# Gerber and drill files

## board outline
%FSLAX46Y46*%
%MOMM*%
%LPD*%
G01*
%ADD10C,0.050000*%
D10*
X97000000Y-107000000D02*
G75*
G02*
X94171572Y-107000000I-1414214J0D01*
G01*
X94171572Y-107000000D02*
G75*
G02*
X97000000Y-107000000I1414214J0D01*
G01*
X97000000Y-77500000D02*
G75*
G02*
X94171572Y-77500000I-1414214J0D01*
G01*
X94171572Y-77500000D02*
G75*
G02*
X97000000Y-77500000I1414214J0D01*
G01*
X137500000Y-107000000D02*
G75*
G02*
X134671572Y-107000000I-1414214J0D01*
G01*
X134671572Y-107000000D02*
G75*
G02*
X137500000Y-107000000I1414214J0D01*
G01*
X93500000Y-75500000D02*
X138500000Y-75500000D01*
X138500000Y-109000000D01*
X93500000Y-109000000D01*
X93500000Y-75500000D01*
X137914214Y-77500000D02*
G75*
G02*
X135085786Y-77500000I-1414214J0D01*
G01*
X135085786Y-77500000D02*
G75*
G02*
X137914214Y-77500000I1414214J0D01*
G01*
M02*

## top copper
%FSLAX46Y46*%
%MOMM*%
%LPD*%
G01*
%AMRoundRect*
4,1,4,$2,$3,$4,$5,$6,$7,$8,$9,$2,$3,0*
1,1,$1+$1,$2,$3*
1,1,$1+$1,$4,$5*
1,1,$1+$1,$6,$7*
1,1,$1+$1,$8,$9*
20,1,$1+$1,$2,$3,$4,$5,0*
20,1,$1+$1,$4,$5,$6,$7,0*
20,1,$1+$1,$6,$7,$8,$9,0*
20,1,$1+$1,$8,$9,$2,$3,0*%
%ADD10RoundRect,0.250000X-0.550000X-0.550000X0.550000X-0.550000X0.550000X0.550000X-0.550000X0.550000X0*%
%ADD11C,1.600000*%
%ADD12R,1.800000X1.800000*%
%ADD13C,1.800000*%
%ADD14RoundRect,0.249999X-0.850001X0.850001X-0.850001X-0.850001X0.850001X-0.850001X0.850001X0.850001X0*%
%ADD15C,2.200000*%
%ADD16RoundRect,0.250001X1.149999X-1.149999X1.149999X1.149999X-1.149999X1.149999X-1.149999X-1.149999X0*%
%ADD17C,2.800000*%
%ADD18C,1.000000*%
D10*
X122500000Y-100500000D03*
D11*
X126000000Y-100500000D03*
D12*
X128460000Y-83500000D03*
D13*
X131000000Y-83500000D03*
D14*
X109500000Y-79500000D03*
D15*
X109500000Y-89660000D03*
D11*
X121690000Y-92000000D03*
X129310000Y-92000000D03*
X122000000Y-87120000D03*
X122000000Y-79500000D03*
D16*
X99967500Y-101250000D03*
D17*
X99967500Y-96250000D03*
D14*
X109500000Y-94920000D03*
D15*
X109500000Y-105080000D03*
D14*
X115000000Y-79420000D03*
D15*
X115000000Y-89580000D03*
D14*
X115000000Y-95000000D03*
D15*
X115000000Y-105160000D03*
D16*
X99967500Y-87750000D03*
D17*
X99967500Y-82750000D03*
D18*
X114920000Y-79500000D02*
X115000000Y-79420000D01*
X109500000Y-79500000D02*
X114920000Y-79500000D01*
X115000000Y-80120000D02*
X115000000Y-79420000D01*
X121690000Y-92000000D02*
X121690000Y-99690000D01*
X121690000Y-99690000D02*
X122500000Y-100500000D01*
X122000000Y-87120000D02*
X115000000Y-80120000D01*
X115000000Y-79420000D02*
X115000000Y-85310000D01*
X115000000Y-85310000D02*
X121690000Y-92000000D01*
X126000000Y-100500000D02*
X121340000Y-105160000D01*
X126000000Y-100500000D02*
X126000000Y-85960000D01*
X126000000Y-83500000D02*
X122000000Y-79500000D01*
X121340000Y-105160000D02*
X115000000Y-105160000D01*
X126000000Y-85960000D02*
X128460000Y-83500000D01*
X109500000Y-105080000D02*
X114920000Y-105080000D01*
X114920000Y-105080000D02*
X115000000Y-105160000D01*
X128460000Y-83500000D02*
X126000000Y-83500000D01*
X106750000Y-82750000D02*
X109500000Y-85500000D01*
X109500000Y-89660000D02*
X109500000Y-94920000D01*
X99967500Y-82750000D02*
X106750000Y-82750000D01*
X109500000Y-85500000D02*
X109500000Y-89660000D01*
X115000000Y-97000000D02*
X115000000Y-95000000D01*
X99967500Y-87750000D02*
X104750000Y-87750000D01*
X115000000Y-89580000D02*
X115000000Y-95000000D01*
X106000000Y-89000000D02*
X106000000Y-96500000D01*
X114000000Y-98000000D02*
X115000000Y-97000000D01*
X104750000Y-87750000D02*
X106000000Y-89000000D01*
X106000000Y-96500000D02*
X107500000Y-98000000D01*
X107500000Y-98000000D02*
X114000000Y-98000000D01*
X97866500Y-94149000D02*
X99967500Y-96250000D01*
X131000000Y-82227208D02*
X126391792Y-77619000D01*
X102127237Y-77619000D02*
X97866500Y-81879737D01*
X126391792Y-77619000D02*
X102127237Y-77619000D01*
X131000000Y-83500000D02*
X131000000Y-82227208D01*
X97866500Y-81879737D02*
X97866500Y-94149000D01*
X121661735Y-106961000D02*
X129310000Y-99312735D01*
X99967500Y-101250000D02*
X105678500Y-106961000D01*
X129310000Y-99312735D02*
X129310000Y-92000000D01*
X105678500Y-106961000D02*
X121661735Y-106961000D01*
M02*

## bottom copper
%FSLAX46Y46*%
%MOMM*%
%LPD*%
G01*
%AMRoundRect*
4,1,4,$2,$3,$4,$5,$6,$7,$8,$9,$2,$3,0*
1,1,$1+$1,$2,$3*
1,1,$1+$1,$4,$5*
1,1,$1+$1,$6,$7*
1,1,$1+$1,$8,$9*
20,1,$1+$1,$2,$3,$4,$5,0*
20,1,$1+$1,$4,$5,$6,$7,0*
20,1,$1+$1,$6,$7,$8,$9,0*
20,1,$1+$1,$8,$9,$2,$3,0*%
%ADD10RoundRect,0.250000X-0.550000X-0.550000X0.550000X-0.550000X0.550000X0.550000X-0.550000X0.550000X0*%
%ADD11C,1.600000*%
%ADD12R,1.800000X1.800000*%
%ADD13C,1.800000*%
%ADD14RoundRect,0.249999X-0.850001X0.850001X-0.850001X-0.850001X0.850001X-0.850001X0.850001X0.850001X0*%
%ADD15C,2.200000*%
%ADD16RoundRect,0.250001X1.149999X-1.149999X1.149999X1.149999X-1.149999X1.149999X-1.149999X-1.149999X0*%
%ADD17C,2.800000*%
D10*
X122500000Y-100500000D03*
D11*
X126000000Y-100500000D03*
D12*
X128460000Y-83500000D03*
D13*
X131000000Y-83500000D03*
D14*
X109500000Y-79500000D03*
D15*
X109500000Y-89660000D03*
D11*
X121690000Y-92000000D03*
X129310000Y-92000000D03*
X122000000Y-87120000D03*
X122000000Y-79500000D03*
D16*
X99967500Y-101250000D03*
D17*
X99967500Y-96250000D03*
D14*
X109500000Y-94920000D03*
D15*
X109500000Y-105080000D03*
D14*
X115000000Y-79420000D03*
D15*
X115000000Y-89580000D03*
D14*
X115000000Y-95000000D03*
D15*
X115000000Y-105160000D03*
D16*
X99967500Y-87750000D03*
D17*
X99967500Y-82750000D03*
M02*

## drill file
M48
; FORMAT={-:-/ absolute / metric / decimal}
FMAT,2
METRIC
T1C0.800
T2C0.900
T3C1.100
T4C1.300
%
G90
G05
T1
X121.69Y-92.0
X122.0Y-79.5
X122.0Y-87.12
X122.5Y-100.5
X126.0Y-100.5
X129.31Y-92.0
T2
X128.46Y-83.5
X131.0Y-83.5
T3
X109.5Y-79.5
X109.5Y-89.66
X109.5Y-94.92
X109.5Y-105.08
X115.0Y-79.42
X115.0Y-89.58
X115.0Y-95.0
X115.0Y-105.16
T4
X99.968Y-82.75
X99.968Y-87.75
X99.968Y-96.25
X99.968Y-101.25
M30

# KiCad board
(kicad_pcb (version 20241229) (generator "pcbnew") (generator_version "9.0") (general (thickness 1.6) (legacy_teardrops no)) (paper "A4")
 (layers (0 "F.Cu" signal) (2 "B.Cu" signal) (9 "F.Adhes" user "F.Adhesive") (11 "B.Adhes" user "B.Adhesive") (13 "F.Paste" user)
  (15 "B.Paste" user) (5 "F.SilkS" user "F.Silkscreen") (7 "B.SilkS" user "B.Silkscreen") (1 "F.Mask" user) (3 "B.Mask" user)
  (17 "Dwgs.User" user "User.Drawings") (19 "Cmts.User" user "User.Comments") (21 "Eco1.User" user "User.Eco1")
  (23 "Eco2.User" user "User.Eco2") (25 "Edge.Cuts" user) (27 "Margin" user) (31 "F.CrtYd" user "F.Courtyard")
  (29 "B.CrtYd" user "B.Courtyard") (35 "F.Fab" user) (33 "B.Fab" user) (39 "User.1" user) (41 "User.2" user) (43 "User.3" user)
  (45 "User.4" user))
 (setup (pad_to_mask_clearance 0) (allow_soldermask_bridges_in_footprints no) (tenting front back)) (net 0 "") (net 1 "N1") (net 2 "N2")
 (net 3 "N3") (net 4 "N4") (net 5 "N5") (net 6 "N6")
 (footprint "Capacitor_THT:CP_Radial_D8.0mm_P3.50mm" (layer "F.Cu") (at 122.5 100.5)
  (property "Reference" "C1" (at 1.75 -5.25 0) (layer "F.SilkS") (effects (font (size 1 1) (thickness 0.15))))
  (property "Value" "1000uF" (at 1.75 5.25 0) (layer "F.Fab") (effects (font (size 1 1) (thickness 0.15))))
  (pad "1" thru_hole roundrect (at 0 0) (size 1.6 1.6) (drill 0.8) (layers "*.Cu" "*.Mask") (remove_unused_layers no)
   (roundrect_rratio 0.15625) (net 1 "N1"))
  (pad "2" thru_hole circle (at 3.5 0) (size 1.6 1.6) (drill 0.8) (layers "*.Cu" "*.Mask") (remove_unused_layers no) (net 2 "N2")))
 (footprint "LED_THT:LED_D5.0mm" (layer "F.Cu") (at 128.46 83.5)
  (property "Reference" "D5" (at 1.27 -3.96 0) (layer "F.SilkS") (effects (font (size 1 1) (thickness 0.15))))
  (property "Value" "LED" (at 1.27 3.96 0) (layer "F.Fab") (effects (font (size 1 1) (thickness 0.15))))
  (pad "1" thru_hole rect (at 0 0) (size 1.8 1.8) (drill 0.9) (layers "*.Cu" "*.Mask") (remove_unused_layers no) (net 2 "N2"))
  (pad "2" thru_hole circle (at 2.54 0) (size 1.8 1.8) (drill 0.9) (layers "*.Cu" "*.Mask") (remove_unused_layers no) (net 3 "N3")))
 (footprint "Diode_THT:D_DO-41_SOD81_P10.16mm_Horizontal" (layer "F.Cu") (at 109.5 79.5 -90)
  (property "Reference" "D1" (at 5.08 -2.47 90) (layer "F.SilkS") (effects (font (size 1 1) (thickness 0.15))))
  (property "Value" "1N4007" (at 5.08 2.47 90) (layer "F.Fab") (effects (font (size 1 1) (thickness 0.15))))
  (pad "1" thru_hole roundrect (at 0 0 270) (size 2.2 2.2) (drill 1.1) (layers "*.Cu" "*.Mask") (remove_unused_layers no)
   (roundrect_rratio 0.113636) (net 1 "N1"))
  (pad "2" thru_hole circle (at 10.16 0 270) (size 2.2 2.2) (drill 1.1) (layers "*.Cu" "*.Mask") (remove_unused_layers no) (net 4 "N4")))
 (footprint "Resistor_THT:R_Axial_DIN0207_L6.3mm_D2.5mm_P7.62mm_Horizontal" (layer "F.Cu") (at 121.69 92)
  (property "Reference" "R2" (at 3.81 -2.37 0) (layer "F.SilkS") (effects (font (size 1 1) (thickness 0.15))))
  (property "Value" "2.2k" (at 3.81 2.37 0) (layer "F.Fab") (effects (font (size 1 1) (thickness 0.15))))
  (pad "1" thru_hole circle (at 0 0) (size 1.6 1.6) (drill 0.8) (layers "*.Cu" "*.Mask") (remove_unused_layers no) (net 1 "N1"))
  (pad "2" thru_hole circle (at 7.62 0) (size 1.6 1.6) (drill 0.8) (layers "*.Cu" "*.Mask") (remove_unused_layers no) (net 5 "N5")))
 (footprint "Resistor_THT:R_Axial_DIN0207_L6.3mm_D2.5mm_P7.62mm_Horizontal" (layer "F.Cu") (at 122 87.12 90)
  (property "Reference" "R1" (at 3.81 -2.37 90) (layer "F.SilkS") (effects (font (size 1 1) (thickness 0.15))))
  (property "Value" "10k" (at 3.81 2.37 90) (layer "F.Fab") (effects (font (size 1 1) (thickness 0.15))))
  (pad "1" thru_hole circle (at 0 0 90) (size 1.6 1.6) (drill 0.8) (layers "*.Cu" "*.Mask") (remove_unused_layers no) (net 1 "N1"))
  (pad "2" thru_hole circle (at 7.62 0 90) (size 1.6 1.6) (drill 0.8) (layers "*.Cu" "*.Mask") (remove_unused_layers no) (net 2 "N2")))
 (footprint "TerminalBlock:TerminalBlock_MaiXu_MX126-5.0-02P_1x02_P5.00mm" (layer "F.Cu") (at 99.9675 101.25 90)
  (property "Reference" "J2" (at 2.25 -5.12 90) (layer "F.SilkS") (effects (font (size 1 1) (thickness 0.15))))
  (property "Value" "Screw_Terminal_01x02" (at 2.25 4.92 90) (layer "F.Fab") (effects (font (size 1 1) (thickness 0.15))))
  (pad "1" thru_hole roundrect (at 0 0 90) (size 2.8 2.8) (drill 1.3) (layers "*.Cu" "*.Mask") (remove_unused_layers no)
   (roundrect_rratio 0.089286) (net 5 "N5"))
  (pad "2" thru_hole circle (at 5 0 90) (size 2.8 2.8) (drill 1.3) (layers "*.Cu" "*.Mask") (remove_unused_layers no) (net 3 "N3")))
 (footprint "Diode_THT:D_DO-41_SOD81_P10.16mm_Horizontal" (layer "F.Cu") (at 109.5 94.92 -90)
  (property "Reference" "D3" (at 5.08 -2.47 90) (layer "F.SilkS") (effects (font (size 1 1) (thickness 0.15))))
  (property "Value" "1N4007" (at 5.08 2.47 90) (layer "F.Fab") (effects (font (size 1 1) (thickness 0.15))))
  (pad "1" thru_hole roundrect (at 0 0 270) (size 2.2 2.2) (drill 1.1) (layers "*.Cu" "*.Mask") (remove_unused_layers no)
   (roundrect_rratio 0.113636) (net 4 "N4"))
  (pad "2" thru_hole circle (at 10.16 0 270) (size 2.2 2.2) (drill 1.1) (layers "*.Cu" "*.Mask") (remove_unused_layers no) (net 2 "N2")))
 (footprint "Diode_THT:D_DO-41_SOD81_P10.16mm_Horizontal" (layer "F.Cu") (at 115 79.42 -90)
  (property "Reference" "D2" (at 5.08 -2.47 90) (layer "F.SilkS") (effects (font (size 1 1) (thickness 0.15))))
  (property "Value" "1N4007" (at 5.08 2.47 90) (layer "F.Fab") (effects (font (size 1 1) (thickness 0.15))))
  (pad "1" thru_hole roundrect (at 0 0 270) (size 2.2 2.2) (drill 1.1) (layers "*.Cu" "*.Mask") (remove_unused_layers no)
   (roundrect_rratio 0.113636) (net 1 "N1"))
  (pad "2" thru_hole circle (at 10.16 0 270) (size 2.2 2.2) (drill 1.1) (layers "*.Cu" "*.Mask") (remove_unused_layers no) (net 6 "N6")))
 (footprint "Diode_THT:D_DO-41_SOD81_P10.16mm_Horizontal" (layer "F.Cu") (at 115 95 -90)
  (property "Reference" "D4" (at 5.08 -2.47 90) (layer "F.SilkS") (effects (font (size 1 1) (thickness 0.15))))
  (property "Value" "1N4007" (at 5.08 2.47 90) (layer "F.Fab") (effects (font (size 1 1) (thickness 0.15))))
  (pad "1" thru_hole roundrect (at 0 0 270) (size 2.2 2.2) (drill 1.1) (layers "*.Cu" "*.Mask") (remove_unused_layers no)
   (roundrect_rratio 0.113636) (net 6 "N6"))
  (pad "2" thru_hole circle (at 10.16 0 270) (size 2.2 2.2) (drill 1.1) (layers "*.Cu" "*.Mask") (remove_unused_layers no) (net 2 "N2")))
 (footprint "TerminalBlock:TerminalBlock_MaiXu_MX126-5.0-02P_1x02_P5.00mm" (layer "F.Cu") (at 99.9675 87.75 90)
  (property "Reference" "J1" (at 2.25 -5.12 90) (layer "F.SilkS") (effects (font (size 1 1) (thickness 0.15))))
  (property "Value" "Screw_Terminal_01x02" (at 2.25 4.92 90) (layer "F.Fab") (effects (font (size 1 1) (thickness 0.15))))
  (pad "1" thru_hole roundrect (at 0 0 90) (size 2.8 2.8) (drill 1.3) (layers "*.Cu" "*.Mask") (remove_unused_layers no)
   (roundrect_rratio 0.089286) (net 6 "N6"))
  (pad "2" thru_hole circle (at 5 0 90) (size 2.8 2.8) (drill 1.3) (layers "*.Cu" "*.Mask") (remove_unused_layers no) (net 4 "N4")))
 (gr_circle (center 95.585786 107) (end 96.585786 108) (stroke (width 0.05) (type default)) (fill no) (layer "Edge.Cuts"))
 (gr_circle (center 95.585786 77.5) (end 96.585786 78.5) (stroke (width 0.05) (type default)) (fill no) (layer "Edge.Cuts"))
 (gr_circle (center 136.085786 107) (end 137.085786 108) (stroke (width 0.05) (type default)) (fill no) (layer "Edge.Cuts"))
 (gr_rect (start 93.5 75.5) (end 138.5 109) (stroke (width 0.05) (type default)) (fill no) (layer "Edge.Cuts"))
 (gr_circle (center 136.5 77.5) (end 137.5 78.5) (stroke (width 0.05) (type default)) (fill no) (layer "Edge.Cuts"))
 (segment (start 114.92 79.5) (end 115 79.42) (width 1) (layer "F.Cu") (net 1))
 (segment (start 109.5 79.5) (end 114.92 79.5) (width 1) (layer "F.Cu") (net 1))
 (segment (start 115 80.12) (end 115 79.42) (width 1) (layer "F.Cu") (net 1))
 (segment (start 121.69 92) (end 121.69 99.69) (width 1) (layer "F.Cu") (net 1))
 (segment (start 121.69 99.69) (end 122.5 100.5) (width 1) (layer "F.Cu") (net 1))
 (segment (start 122 87.12) (end 115 80.12) (width 1) (layer "F.Cu") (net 1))
 (segment (start 115 79.42) (end 115 85.31) (width 1) (layer "F.Cu") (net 1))
 (segment (start 115 85.31) (end 121.69 92) (width 1) (layer "F.Cu") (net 1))
 (segment (start 126 100.5) (end 121.34 105.16) (width 1) (layer "F.Cu") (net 2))
 (segment (start 126 100.5) (end 126 85.96) (width 1) (layer "F.Cu") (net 2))
 (segment (start 126 83.5) (end 122 79.5) (width 1) (layer "F.Cu") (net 2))
 (segment (start 121.34 105.16) (end 115 105.16) (width 1) (layer "F.Cu") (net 2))
 (segment (start 126 85.96) (end 128.46 83.5) (width 1) (layer "F.Cu") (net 2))
 (segment (start 109.5 105.08) (end 114.92 105.08) (width 1) (layer "F.Cu") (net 2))
 (segment (start 114.92 105.08) (end 115 105.16) (width 1) (layer "F.Cu") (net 2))
 (segment (start 128.46 83.5) (end 126 83.5) (width 1) (layer "F.Cu") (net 2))
 (segment (start 106.75 82.75) (end 109.5 85.5) (width 1) (layer "F.Cu") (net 4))
 (segment (start 109.5 89.66) (end 109.5 94.92) (width 1) (layer "F.Cu") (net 4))
 (segment (start 99.9675 82.75) (end 106.75 82.75) (width 1) (layer "F.Cu") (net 4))
 (segment (start 109.5 85.5) (end 109.5 89.66) (width 1) (layer "F.Cu") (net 4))
 (segment (start 115 97) (end 115 95) (width 1) (layer "F.Cu") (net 6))
 (segment (start 99.9675 87.75) (end 104.75 87.75) (width 1) (layer "F.Cu") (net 6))
 (segment (start 115 89.58) (end 115 95) (width 1) (layer "F.Cu") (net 6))
 (segment (start 106 89) (end 106 96.5) (width 1) (layer "F.Cu") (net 6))
 (segment (start 114 98) (end 115 97) (width 1) (layer "F.Cu") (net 6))
 (segment (start 104.75 87.75) (end 106 89) (width 1) (layer "F.Cu") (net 6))
 (segment (start 106 96.5) (end 107.5 98) (width 1) (layer "F.Cu") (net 6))
 (segment (start 107.5 98) (end 114 98) (width 1) (layer "F.Cu") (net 6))
 (segment (start 97.8665 94.149) (end 99.9675 96.25) (width 1) (layer "F.Cu") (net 3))
 (segment (start 131 82.227208) (end 126.391792 77.619) (width 1) (layer "F.Cu") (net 3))
 (segment (start 102.127237 77.619) (end 97.8665 81.879737) (width 1) (layer "F.Cu") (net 3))
 (segment (start 126.391792 77.619) (end 102.127237 77.619) (width 1) (layer "F.Cu") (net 3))
 (segment (start 131 83.5) (end 131 82.227208) (width 1) (layer "F.Cu") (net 3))
 (segment (start 97.8665 81.879737) (end 97.8665 94.149) (width 1) (layer "F.Cu") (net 3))
 (segment (start 121.661735 106.961) (end 129.31 99.312735) (width 1) (layer "F.Cu") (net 5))
 (segment (start 99.9675 101.25) (end 105.6785 106.961) (width 1) (layer "F.Cu") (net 5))
 (segment (start 129.31 99.312735) (end 129.31 92) (width 1) (layer "F.Cu") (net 5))
 (segment (start 105.6785 106.961) (end 121.661735 106.961) (width 1) (layer "F.Cu") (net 5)))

